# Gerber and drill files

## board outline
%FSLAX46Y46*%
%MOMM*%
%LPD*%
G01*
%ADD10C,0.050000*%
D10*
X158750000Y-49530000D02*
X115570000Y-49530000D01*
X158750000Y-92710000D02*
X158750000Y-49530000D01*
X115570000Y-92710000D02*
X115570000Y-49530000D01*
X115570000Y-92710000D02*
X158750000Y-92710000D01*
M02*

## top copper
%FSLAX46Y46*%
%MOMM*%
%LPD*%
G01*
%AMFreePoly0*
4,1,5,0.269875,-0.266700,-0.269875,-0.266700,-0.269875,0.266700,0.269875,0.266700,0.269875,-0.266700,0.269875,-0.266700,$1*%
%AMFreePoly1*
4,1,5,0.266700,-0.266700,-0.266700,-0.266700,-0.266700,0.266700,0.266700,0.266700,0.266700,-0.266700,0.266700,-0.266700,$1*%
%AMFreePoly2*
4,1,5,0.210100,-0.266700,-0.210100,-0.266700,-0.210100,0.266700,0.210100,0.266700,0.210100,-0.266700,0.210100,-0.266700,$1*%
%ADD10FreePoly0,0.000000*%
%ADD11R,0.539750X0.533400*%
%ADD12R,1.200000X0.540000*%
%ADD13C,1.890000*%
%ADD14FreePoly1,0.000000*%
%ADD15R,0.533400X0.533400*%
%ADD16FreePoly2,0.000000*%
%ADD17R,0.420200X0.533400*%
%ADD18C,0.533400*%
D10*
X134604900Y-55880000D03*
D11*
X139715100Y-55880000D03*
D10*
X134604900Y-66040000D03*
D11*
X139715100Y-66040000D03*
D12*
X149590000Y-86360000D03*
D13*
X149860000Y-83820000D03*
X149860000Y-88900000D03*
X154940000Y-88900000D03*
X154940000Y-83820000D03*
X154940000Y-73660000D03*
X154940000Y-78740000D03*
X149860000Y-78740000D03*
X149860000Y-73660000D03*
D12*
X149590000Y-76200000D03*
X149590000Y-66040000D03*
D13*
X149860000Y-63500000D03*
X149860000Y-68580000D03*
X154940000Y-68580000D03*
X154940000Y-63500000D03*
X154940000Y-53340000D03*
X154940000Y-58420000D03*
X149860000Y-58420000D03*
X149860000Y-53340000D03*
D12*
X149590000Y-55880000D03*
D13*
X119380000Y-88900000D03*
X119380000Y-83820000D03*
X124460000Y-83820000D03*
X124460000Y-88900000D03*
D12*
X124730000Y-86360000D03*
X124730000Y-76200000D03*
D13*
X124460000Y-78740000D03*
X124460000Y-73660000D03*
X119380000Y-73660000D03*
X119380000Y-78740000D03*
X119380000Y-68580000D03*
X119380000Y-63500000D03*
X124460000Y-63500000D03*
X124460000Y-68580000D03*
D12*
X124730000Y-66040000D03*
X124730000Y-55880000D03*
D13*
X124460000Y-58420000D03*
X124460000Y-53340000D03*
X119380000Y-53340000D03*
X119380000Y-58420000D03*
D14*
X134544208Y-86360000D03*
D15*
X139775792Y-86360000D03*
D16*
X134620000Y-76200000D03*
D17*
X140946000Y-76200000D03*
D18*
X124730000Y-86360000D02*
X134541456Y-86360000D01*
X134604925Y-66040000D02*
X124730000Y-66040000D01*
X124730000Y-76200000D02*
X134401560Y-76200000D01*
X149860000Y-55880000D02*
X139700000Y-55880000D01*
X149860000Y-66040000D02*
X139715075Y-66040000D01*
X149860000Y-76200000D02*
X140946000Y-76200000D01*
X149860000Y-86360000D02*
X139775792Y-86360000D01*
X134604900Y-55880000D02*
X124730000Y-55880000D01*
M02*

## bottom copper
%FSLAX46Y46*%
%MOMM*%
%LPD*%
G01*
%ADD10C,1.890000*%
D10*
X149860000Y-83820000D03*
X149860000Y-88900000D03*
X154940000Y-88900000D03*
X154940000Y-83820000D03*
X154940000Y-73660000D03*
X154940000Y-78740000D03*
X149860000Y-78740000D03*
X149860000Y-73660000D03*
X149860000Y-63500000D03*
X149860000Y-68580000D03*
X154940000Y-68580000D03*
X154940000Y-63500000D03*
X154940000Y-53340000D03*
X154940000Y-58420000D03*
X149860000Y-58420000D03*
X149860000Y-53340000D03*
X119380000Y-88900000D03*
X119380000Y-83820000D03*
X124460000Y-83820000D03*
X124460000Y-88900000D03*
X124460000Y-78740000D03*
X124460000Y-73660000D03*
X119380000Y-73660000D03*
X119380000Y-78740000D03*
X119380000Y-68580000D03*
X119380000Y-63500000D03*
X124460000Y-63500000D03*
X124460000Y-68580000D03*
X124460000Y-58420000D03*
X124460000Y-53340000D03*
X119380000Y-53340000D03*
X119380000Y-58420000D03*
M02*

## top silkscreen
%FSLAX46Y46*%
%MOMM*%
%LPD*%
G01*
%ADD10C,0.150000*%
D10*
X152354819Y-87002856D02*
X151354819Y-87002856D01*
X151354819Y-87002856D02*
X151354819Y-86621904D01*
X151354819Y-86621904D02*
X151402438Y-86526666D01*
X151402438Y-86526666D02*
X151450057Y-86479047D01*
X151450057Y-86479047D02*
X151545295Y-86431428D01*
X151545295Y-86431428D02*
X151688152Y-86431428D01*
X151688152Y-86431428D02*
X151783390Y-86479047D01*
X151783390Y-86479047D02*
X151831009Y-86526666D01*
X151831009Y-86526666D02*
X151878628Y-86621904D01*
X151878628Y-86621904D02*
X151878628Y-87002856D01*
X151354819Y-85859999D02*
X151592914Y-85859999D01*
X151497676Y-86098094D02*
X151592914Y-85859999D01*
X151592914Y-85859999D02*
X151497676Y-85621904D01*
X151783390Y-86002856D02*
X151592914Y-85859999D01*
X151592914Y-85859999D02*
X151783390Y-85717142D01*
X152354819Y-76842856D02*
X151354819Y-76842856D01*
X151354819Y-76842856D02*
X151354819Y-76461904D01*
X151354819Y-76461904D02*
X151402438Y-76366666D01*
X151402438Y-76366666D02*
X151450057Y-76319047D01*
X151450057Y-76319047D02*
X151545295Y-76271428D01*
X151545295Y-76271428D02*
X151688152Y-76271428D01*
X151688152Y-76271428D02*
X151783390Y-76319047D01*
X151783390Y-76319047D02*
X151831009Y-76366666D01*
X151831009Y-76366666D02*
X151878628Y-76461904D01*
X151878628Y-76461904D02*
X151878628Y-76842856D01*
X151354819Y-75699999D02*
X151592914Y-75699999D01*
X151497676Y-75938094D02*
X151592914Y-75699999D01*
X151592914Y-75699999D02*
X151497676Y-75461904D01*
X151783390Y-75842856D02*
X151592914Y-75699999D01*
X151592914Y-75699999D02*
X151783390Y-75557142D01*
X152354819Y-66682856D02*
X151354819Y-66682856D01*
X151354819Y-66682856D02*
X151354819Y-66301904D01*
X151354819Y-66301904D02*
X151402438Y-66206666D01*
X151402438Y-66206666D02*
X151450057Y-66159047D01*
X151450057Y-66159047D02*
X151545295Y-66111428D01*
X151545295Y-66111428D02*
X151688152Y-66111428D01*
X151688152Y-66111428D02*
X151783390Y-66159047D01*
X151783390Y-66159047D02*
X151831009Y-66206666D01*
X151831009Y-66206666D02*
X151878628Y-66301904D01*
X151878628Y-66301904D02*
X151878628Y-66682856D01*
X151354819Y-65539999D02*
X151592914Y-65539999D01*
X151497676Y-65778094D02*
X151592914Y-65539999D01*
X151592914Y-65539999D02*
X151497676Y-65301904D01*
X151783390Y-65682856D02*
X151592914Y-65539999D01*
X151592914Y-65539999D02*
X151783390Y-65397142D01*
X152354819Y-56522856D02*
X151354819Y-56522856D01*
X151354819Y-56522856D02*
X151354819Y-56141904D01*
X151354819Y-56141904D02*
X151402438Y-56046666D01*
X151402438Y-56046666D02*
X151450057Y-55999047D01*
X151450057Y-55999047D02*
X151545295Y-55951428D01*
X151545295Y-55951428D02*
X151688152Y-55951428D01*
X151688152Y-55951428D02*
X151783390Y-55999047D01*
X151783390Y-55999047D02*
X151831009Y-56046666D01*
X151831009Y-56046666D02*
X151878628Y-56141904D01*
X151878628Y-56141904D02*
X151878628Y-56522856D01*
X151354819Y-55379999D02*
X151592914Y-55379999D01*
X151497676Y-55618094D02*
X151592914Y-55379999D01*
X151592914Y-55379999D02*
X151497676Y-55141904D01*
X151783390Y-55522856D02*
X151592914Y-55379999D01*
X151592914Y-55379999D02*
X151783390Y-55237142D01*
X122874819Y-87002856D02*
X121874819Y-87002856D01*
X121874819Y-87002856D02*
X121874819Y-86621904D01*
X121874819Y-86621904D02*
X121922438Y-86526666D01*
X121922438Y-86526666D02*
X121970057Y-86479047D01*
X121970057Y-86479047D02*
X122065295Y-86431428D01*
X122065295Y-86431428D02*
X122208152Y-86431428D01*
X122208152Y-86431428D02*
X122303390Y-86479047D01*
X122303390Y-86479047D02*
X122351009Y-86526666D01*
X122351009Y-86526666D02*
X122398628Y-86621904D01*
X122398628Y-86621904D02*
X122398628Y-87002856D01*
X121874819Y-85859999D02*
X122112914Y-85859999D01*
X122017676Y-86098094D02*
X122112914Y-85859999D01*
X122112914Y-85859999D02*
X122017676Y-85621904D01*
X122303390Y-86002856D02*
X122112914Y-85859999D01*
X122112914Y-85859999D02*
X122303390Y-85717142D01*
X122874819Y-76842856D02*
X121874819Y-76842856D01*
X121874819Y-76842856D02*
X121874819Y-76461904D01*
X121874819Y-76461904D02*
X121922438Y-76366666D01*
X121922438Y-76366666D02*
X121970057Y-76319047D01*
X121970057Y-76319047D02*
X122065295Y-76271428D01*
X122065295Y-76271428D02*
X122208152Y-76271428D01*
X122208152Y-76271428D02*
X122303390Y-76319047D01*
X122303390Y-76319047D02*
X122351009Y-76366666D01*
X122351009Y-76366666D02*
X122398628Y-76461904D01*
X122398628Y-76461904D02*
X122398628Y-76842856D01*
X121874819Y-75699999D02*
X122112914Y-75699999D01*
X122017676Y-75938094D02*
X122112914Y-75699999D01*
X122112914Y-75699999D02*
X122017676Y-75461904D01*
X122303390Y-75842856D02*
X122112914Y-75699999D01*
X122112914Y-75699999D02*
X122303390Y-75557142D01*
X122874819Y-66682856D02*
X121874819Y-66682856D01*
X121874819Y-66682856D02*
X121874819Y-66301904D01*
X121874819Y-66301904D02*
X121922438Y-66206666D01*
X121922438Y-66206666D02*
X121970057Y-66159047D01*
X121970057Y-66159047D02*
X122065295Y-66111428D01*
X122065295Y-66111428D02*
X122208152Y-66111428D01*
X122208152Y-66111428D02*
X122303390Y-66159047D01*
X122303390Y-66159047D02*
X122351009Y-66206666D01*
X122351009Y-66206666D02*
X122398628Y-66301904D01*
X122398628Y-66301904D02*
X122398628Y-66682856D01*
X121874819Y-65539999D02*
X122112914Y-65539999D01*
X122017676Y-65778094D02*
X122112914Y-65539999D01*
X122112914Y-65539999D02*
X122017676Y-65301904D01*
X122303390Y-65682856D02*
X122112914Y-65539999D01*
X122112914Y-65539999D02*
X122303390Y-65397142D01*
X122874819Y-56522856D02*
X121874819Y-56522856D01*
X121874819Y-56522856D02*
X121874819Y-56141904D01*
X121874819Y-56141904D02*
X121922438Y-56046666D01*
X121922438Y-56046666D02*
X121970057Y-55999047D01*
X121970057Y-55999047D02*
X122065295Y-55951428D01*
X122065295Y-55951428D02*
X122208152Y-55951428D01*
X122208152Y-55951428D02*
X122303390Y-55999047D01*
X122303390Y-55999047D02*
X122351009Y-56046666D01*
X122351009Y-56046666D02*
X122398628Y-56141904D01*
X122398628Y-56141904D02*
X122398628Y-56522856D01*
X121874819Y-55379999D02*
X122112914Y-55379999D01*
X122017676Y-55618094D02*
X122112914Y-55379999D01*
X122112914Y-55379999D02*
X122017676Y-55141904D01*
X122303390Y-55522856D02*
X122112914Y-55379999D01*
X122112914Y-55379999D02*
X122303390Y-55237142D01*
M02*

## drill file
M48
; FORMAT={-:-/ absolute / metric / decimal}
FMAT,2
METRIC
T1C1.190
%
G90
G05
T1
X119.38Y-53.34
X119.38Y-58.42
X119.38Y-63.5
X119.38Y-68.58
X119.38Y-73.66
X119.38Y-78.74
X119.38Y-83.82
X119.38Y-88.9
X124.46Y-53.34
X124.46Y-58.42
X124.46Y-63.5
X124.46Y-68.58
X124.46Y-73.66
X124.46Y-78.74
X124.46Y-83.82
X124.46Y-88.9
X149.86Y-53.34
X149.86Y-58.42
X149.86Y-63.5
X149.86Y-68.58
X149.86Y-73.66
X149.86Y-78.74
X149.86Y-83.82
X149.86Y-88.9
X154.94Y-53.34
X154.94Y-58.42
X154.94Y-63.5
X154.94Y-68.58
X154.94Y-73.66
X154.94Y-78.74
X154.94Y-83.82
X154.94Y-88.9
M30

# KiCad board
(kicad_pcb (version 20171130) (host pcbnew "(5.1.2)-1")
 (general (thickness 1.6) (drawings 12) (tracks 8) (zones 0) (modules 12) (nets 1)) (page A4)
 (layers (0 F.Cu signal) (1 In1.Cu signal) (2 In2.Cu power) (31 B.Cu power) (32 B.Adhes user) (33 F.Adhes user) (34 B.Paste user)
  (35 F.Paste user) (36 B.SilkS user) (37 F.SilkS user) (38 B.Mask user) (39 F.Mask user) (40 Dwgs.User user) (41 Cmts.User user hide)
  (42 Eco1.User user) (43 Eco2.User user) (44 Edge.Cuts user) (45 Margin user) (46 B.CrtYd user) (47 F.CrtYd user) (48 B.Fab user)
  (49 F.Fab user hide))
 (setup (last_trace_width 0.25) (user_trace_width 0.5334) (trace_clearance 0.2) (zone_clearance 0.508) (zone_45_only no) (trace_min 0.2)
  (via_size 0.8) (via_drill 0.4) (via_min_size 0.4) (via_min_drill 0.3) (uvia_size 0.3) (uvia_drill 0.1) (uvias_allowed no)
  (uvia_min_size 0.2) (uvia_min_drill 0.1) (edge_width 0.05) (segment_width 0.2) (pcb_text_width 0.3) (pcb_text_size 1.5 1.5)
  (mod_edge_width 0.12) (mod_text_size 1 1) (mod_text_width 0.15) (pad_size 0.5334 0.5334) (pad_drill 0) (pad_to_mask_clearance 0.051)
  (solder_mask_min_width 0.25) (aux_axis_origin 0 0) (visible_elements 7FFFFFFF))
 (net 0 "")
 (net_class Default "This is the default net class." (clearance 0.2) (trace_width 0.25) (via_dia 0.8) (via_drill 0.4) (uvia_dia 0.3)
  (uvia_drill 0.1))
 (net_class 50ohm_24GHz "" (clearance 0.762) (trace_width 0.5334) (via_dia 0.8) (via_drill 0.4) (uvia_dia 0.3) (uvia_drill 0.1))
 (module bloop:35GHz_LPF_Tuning (layer F.Cu) (at 137.16 55.88)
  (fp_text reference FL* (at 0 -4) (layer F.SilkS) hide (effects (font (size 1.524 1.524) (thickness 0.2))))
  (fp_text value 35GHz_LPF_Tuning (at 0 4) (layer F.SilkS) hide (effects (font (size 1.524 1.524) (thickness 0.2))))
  (pad 1 smd custom (at -2.5551 0) (size 0.53975 0.5334) (layers F.Cu F.Paste F.Mask) (solder_mask_margin 0.00001)
   (solder_paste_margin 0.00001) (clearance 0.00001) (zone_connect 0) (options (clearance outline) (anchor rect)) (primitives))
  (pad 1 smd rect (at 2.5551 0) (size 0.53975 0.5334) (layers F.Cu F.Paste F.Mask) (solder_mask_margin 0.00001)
   (solder_paste_margin 0.00001) (solder_paste_margin_ratio -0.000000001) (clearance 0.00001) (zone_connect 0)))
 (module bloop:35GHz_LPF (layer F.Cu) (at 137.16 66.04)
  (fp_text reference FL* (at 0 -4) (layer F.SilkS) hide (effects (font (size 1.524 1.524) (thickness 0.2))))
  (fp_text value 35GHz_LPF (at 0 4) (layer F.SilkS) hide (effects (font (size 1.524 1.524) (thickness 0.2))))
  (pad 1 smd custom (at -2.5551 0) (size 0.53975 0.5334) (layers F.Cu F.Paste F.Mask) (solder_mask_margin 0.00001)
   (solder_paste_margin 0.00001) (clearance 0.00001) (zone_connect 0) (options (clearance outline) (anchor rect)) (primitives))
  (pad 1 smd rect (at 2.5551 0) (size 0.53975 0.5334) (layers F.Cu F.Paste F.Mask) (solder_mask_margin 0.00001)
   (solder_paste_margin 0.00001) (clearance 0.00001)))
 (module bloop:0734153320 (layer F.Cu) (at 152.4 86.36 270)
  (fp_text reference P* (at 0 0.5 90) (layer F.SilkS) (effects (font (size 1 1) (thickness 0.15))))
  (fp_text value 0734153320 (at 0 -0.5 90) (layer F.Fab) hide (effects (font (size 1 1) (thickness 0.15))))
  (pad 1 smd rect (at 0 2.81 270) (size 0.54 1.2) (layers F.Cu F.Paste F.Mask))
  (pad 2 thru_hole circle (at -2.54 2.54 270) (size 1.89 1.89) (drill 1.19) (layers *.Cu *.Mask))
  (pad 2 thru_hole circle (at 2.54 2.54 270) (size 1.89 1.89) (drill 1.19) (layers *.Cu *.Mask))
  (pad 2 thru_hole circle (at 2.54 -2.54 270) (size 1.89 1.89) (drill 1.19) (layers *.Cu *.Mask))
  (pad 2 thru_hole circle (at -2.54 -2.54 270) (size 1.89 1.89) (drill 1.19) (layers *.Cu *.Mask)))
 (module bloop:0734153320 (layer F.Cu) (at 152.4 76.2 270)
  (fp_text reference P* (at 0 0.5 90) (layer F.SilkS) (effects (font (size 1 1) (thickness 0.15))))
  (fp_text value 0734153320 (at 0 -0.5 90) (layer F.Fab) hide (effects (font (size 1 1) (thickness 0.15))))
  (pad 2 thru_hole circle (at -2.54 -2.54 270) (size 1.89 1.89) (drill 1.19) (layers *.Cu *.Mask))
  (pad 2 thru_hole circle (at 2.54 -2.54 270) (size 1.89 1.89) (drill 1.19) (layers *.Cu *.Mask))
  (pad 2 thru_hole circle (at 2.54 2.54 270) (size 1.89 1.89) (drill 1.19) (layers *.Cu *.Mask))
  (pad 2 thru_hole circle (at -2.54 2.54 270) (size 1.89 1.89) (drill 1.19) (layers *.Cu *.Mask))
  (pad 1 smd rect (at 0 2.81 270) (size 0.54 1.2) (layers F.Cu F.Paste F.Mask)))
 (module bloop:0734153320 (layer F.Cu) (at 152.4 66.04 270)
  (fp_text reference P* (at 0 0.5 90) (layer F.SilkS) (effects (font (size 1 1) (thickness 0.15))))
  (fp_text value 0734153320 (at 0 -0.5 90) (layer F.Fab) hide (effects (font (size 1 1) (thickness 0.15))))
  (pad 1 smd rect (at 0 2.81 270) (size 0.54 1.2) (layers F.Cu F.Paste F.Mask))
  (pad 2 thru_hole circle (at -2.54 2.54 270) (size 1.89 1.89) (drill 1.19) (layers *.Cu *.Mask))
  (pad 2 thru_hole circle (at 2.54 2.54 270) (size 1.89 1.89) (drill 1.19) (layers *.Cu *.Mask))
  (pad 2 thru_hole circle (at 2.54 -2.54 270) (size 1.89 1.89) (drill 1.19) (layers *.Cu *.Mask))
  (pad 2 thru_hole circle (at -2.54 -2.54 270) (size 1.89 1.89) (drill 1.19) (layers *.Cu *.Mask)))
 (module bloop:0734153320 (layer F.Cu) (at 152.4 55.88 270)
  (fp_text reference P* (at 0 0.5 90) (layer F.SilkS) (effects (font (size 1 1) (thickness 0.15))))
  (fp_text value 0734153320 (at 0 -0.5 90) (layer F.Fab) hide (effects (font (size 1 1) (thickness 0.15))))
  (pad 2 thru_hole circle (at -2.54 -2.54 270) (size 1.89 1.89) (drill 1.19) (layers *.Cu *.Mask))
  (pad 2 thru_hole circle (at 2.54 -2.54 270) (size 1.89 1.89) (drill 1.19) (layers *.Cu *.Mask))
  (pad 2 thru_hole circle (at 2.54 2.54 270) (size 1.89 1.89) (drill 1.19) (layers *.Cu *.Mask))
  (pad 2 thru_hole circle (at -2.54 2.54 270) (size 1.89 1.89) (drill 1.19) (layers *.Cu *.Mask))
  (pad 1 smd rect (at 0 2.81 270) (size 0.54 1.2) (layers F.Cu F.Paste F.Mask)))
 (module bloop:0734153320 (layer F.Cu) (at 121.92 86.36 90)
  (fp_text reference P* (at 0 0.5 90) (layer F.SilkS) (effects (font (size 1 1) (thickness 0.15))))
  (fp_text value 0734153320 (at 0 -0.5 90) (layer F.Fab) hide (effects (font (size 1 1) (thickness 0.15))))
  (pad 2 thru_hole circle (at -2.54 -2.54 90) (size 1.89 1.89) (drill 1.19) (layers *.Cu *.Mask))
  (pad 2 thru_hole circle (at 2.54 -2.54 90) (size 1.89 1.89) (drill 1.19) (layers *.Cu *.Mask))
  (pad 2 thru_hole circle (at 2.54 2.54 90) (size 1.89 1.89) (drill 1.19) (layers *.Cu *.Mask))
  (pad 2 thru_hole circle (at -2.54 2.54 90) (size 1.89 1.89) (drill 1.19) (layers *.Cu *.Mask))
  (pad 1 smd rect (at 0 2.81 90) (size 0.54 1.2) (layers F.Cu F.Paste F.Mask)))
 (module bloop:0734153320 (layer F.Cu) (at 121.92 76.2 90)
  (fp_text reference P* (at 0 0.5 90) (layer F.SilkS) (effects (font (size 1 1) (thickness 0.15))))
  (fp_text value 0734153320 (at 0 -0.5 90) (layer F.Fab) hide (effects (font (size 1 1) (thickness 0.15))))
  (pad 1 smd rect (at 0 2.81 90) (size 0.54 1.2) (layers F.Cu F.Paste F.Mask))
  (pad 2 thru_hole circle (at -2.54 2.54 90) (size 1.89 1.89) (drill 1.19) (layers *.Cu *.Mask))
  (pad 2 thru_hole circle (at 2.54 2.54 90) (size 1.89 1.89) (drill 1.19) (layers *.Cu *.Mask))
  (pad 2 thru_hole circle (at 2.54 -2.54 90) (size 1.89 1.89) (drill 1.19) (layers *.Cu *.Mask))
  (pad 2 thru_hole circle (at -2.54 -2.54 90) (size 1.89 1.89) (drill 1.19) (layers *.Cu *.Mask)))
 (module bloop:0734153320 (layer F.Cu) (at 121.92 66.04 90)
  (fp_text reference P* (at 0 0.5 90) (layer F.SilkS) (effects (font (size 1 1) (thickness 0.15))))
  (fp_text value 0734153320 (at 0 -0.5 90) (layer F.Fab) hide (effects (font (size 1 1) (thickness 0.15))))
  (pad 2 thru_hole circle (at -2.54 -2.54 90) (size 1.89 1.89) (drill 1.19) (layers *.Cu *.Mask))
  (pad 2 thru_hole circle (at 2.54 -2.54 90) (size 1.89 1.89) (drill 1.19) (layers *.Cu *.Mask))
  (pad 2 thru_hole circle (at 2.54 2.54 90) (size 1.89 1.89) (drill 1.19) (layers *.Cu *.Mask))
  (pad 2 thru_hole circle (at -2.54 2.54 90) (size 1.89 1.89) (drill 1.19) (layers *.Cu *.Mask))
  (pad 1 smd rect (at 0 2.81 90) (size 0.54 1.2) (layers F.Cu F.Paste F.Mask)))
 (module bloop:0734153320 (layer F.Cu) (at 121.92 55.88 90)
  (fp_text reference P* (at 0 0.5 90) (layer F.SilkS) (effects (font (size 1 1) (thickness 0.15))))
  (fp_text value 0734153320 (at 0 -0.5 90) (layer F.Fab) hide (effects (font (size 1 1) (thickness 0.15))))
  (pad 1 smd rect (at 0 2.81 90) (size 0.54 1.2) (layers F.Cu F.Paste F.Mask))
  (pad 2 thru_hole circle (at -2.54 2.54 90) (size 1.89 1.89) (drill 1.19) (layers *.Cu *.Mask))
  (pad 2 thru_hole circle (at 2.54 2.54 90) (size 1.89 1.89) (drill 1.19) (layers *.Cu *.Mask))
  (pad 2 thru_hole circle (at 2.54 -2.54 90) (size 1.89 1.89) (drill 1.19) (layers *.Cu *.Mask))
  (pad 2 thru_hole circle (at -2.54 -2.54 90) (size 1.89 1.89) (drill 1.19) (layers *.Cu *.Mask)))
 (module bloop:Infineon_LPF (layer F.Cu) (at 137.16 86.362752)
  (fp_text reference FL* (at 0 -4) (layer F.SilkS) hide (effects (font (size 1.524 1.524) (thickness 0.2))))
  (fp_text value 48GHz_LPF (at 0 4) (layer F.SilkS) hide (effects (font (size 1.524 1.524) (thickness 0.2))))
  (pad 1 smd custom (at -2.615792 -0.002752) (size 0.5334 0.5334) (layers F.Cu F.Paste F.Mask) (solder_mask_margin 0.000001)
   (solder_paste_margin -0.000001) (solder_paste_margin_ratio -0.00000001) (clearance 0.000001) (zone_connect 0)
   (options (clearance outline) (anchor rect)) (primitives))
  (pad 1 smd rect (at 2.615792 -0.002752) (size 0.5334 0.5334) (layers F.Cu F.Paste F.Mask) (solder_mask_margin 0.000001)
   (solder_paste_margin -0.000001) (solder_paste_margin_ratio -0.00000001) (clearance 0.000001)))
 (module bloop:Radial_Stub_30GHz (layer F.Cu) (at 134.62 76.2)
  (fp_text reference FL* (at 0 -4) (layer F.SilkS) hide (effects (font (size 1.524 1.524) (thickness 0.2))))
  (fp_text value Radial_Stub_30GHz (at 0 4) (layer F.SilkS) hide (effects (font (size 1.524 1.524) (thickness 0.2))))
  (pad 1 smd custom (at 0 0) (size 0.4202 0.5334) (layers F.Cu F.Paste F.Mask) (solder_mask_margin 0.000001) (solder_paste_margin -0.000001)
   (solder_paste_margin_ratio -0.00000001) (clearance 0.000001) (zone_connect 0) (options (clearance outline) (anchor rect)) (primitives))
  (pad 1 smd rect (at 6.326 0) (size 0.4202 0.5334) (layers F.Cu F.Paste F.Mask) (solder_mask_margin 0.000001)
   (solder_paste_margin -0.000001) (solder_paste_margin_ratio -0.00000001) (clearance 0.000001) (zone_connect 0)))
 (gr_line (start 158.75 49.53) (end 115.57 49.53) (layer Edge.Cuts) (width 0.05))
 (gr_line (start 158.75 92.71) (end 158.75 49.53) (layer Edge.Cuts) (width 0.05))
 (gr_line (start 115.57 92.71) (end 115.57 49.53) (layer Edge.Cuts) (width 0.05))
 (gr_line (start 115.57 92.71) (end 158.75 92.71) (layer Edge.Cuts) (width 0.05))
 (segment (start 124.73 86.36) (end 134.541456 86.36) (width 0.5334) (layer F.Cu) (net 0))
 (segment (start 134.604925 66.04) (end 124.73 66.04) (width 0.5334) (layer F.Cu) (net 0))
 (segment (start 124.73 76.2) (end 134.40156 76.2) (width 0.5334) (layer F.Cu) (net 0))
 (segment (start 149.86 55.88) (end 139.7 55.88) (width 0.5334) (layer F.Cu) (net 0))
 (segment (start 149.86 66.04) (end 139.715075 66.04) (width 0.5334) (layer F.Cu) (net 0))
 (segment (start 149.86 76.2) (end 140.946 76.2) (width 0.5334) (layer F.Cu) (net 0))
 (segment (start 149.86 86.36) (end 139.775792 86.36) (width 0.5334) (layer F.Cu) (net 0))
 (segment (start 134.6049 55.88) (end 124.73 55.88) (width 0.5334) (layer F.Cu) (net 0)))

